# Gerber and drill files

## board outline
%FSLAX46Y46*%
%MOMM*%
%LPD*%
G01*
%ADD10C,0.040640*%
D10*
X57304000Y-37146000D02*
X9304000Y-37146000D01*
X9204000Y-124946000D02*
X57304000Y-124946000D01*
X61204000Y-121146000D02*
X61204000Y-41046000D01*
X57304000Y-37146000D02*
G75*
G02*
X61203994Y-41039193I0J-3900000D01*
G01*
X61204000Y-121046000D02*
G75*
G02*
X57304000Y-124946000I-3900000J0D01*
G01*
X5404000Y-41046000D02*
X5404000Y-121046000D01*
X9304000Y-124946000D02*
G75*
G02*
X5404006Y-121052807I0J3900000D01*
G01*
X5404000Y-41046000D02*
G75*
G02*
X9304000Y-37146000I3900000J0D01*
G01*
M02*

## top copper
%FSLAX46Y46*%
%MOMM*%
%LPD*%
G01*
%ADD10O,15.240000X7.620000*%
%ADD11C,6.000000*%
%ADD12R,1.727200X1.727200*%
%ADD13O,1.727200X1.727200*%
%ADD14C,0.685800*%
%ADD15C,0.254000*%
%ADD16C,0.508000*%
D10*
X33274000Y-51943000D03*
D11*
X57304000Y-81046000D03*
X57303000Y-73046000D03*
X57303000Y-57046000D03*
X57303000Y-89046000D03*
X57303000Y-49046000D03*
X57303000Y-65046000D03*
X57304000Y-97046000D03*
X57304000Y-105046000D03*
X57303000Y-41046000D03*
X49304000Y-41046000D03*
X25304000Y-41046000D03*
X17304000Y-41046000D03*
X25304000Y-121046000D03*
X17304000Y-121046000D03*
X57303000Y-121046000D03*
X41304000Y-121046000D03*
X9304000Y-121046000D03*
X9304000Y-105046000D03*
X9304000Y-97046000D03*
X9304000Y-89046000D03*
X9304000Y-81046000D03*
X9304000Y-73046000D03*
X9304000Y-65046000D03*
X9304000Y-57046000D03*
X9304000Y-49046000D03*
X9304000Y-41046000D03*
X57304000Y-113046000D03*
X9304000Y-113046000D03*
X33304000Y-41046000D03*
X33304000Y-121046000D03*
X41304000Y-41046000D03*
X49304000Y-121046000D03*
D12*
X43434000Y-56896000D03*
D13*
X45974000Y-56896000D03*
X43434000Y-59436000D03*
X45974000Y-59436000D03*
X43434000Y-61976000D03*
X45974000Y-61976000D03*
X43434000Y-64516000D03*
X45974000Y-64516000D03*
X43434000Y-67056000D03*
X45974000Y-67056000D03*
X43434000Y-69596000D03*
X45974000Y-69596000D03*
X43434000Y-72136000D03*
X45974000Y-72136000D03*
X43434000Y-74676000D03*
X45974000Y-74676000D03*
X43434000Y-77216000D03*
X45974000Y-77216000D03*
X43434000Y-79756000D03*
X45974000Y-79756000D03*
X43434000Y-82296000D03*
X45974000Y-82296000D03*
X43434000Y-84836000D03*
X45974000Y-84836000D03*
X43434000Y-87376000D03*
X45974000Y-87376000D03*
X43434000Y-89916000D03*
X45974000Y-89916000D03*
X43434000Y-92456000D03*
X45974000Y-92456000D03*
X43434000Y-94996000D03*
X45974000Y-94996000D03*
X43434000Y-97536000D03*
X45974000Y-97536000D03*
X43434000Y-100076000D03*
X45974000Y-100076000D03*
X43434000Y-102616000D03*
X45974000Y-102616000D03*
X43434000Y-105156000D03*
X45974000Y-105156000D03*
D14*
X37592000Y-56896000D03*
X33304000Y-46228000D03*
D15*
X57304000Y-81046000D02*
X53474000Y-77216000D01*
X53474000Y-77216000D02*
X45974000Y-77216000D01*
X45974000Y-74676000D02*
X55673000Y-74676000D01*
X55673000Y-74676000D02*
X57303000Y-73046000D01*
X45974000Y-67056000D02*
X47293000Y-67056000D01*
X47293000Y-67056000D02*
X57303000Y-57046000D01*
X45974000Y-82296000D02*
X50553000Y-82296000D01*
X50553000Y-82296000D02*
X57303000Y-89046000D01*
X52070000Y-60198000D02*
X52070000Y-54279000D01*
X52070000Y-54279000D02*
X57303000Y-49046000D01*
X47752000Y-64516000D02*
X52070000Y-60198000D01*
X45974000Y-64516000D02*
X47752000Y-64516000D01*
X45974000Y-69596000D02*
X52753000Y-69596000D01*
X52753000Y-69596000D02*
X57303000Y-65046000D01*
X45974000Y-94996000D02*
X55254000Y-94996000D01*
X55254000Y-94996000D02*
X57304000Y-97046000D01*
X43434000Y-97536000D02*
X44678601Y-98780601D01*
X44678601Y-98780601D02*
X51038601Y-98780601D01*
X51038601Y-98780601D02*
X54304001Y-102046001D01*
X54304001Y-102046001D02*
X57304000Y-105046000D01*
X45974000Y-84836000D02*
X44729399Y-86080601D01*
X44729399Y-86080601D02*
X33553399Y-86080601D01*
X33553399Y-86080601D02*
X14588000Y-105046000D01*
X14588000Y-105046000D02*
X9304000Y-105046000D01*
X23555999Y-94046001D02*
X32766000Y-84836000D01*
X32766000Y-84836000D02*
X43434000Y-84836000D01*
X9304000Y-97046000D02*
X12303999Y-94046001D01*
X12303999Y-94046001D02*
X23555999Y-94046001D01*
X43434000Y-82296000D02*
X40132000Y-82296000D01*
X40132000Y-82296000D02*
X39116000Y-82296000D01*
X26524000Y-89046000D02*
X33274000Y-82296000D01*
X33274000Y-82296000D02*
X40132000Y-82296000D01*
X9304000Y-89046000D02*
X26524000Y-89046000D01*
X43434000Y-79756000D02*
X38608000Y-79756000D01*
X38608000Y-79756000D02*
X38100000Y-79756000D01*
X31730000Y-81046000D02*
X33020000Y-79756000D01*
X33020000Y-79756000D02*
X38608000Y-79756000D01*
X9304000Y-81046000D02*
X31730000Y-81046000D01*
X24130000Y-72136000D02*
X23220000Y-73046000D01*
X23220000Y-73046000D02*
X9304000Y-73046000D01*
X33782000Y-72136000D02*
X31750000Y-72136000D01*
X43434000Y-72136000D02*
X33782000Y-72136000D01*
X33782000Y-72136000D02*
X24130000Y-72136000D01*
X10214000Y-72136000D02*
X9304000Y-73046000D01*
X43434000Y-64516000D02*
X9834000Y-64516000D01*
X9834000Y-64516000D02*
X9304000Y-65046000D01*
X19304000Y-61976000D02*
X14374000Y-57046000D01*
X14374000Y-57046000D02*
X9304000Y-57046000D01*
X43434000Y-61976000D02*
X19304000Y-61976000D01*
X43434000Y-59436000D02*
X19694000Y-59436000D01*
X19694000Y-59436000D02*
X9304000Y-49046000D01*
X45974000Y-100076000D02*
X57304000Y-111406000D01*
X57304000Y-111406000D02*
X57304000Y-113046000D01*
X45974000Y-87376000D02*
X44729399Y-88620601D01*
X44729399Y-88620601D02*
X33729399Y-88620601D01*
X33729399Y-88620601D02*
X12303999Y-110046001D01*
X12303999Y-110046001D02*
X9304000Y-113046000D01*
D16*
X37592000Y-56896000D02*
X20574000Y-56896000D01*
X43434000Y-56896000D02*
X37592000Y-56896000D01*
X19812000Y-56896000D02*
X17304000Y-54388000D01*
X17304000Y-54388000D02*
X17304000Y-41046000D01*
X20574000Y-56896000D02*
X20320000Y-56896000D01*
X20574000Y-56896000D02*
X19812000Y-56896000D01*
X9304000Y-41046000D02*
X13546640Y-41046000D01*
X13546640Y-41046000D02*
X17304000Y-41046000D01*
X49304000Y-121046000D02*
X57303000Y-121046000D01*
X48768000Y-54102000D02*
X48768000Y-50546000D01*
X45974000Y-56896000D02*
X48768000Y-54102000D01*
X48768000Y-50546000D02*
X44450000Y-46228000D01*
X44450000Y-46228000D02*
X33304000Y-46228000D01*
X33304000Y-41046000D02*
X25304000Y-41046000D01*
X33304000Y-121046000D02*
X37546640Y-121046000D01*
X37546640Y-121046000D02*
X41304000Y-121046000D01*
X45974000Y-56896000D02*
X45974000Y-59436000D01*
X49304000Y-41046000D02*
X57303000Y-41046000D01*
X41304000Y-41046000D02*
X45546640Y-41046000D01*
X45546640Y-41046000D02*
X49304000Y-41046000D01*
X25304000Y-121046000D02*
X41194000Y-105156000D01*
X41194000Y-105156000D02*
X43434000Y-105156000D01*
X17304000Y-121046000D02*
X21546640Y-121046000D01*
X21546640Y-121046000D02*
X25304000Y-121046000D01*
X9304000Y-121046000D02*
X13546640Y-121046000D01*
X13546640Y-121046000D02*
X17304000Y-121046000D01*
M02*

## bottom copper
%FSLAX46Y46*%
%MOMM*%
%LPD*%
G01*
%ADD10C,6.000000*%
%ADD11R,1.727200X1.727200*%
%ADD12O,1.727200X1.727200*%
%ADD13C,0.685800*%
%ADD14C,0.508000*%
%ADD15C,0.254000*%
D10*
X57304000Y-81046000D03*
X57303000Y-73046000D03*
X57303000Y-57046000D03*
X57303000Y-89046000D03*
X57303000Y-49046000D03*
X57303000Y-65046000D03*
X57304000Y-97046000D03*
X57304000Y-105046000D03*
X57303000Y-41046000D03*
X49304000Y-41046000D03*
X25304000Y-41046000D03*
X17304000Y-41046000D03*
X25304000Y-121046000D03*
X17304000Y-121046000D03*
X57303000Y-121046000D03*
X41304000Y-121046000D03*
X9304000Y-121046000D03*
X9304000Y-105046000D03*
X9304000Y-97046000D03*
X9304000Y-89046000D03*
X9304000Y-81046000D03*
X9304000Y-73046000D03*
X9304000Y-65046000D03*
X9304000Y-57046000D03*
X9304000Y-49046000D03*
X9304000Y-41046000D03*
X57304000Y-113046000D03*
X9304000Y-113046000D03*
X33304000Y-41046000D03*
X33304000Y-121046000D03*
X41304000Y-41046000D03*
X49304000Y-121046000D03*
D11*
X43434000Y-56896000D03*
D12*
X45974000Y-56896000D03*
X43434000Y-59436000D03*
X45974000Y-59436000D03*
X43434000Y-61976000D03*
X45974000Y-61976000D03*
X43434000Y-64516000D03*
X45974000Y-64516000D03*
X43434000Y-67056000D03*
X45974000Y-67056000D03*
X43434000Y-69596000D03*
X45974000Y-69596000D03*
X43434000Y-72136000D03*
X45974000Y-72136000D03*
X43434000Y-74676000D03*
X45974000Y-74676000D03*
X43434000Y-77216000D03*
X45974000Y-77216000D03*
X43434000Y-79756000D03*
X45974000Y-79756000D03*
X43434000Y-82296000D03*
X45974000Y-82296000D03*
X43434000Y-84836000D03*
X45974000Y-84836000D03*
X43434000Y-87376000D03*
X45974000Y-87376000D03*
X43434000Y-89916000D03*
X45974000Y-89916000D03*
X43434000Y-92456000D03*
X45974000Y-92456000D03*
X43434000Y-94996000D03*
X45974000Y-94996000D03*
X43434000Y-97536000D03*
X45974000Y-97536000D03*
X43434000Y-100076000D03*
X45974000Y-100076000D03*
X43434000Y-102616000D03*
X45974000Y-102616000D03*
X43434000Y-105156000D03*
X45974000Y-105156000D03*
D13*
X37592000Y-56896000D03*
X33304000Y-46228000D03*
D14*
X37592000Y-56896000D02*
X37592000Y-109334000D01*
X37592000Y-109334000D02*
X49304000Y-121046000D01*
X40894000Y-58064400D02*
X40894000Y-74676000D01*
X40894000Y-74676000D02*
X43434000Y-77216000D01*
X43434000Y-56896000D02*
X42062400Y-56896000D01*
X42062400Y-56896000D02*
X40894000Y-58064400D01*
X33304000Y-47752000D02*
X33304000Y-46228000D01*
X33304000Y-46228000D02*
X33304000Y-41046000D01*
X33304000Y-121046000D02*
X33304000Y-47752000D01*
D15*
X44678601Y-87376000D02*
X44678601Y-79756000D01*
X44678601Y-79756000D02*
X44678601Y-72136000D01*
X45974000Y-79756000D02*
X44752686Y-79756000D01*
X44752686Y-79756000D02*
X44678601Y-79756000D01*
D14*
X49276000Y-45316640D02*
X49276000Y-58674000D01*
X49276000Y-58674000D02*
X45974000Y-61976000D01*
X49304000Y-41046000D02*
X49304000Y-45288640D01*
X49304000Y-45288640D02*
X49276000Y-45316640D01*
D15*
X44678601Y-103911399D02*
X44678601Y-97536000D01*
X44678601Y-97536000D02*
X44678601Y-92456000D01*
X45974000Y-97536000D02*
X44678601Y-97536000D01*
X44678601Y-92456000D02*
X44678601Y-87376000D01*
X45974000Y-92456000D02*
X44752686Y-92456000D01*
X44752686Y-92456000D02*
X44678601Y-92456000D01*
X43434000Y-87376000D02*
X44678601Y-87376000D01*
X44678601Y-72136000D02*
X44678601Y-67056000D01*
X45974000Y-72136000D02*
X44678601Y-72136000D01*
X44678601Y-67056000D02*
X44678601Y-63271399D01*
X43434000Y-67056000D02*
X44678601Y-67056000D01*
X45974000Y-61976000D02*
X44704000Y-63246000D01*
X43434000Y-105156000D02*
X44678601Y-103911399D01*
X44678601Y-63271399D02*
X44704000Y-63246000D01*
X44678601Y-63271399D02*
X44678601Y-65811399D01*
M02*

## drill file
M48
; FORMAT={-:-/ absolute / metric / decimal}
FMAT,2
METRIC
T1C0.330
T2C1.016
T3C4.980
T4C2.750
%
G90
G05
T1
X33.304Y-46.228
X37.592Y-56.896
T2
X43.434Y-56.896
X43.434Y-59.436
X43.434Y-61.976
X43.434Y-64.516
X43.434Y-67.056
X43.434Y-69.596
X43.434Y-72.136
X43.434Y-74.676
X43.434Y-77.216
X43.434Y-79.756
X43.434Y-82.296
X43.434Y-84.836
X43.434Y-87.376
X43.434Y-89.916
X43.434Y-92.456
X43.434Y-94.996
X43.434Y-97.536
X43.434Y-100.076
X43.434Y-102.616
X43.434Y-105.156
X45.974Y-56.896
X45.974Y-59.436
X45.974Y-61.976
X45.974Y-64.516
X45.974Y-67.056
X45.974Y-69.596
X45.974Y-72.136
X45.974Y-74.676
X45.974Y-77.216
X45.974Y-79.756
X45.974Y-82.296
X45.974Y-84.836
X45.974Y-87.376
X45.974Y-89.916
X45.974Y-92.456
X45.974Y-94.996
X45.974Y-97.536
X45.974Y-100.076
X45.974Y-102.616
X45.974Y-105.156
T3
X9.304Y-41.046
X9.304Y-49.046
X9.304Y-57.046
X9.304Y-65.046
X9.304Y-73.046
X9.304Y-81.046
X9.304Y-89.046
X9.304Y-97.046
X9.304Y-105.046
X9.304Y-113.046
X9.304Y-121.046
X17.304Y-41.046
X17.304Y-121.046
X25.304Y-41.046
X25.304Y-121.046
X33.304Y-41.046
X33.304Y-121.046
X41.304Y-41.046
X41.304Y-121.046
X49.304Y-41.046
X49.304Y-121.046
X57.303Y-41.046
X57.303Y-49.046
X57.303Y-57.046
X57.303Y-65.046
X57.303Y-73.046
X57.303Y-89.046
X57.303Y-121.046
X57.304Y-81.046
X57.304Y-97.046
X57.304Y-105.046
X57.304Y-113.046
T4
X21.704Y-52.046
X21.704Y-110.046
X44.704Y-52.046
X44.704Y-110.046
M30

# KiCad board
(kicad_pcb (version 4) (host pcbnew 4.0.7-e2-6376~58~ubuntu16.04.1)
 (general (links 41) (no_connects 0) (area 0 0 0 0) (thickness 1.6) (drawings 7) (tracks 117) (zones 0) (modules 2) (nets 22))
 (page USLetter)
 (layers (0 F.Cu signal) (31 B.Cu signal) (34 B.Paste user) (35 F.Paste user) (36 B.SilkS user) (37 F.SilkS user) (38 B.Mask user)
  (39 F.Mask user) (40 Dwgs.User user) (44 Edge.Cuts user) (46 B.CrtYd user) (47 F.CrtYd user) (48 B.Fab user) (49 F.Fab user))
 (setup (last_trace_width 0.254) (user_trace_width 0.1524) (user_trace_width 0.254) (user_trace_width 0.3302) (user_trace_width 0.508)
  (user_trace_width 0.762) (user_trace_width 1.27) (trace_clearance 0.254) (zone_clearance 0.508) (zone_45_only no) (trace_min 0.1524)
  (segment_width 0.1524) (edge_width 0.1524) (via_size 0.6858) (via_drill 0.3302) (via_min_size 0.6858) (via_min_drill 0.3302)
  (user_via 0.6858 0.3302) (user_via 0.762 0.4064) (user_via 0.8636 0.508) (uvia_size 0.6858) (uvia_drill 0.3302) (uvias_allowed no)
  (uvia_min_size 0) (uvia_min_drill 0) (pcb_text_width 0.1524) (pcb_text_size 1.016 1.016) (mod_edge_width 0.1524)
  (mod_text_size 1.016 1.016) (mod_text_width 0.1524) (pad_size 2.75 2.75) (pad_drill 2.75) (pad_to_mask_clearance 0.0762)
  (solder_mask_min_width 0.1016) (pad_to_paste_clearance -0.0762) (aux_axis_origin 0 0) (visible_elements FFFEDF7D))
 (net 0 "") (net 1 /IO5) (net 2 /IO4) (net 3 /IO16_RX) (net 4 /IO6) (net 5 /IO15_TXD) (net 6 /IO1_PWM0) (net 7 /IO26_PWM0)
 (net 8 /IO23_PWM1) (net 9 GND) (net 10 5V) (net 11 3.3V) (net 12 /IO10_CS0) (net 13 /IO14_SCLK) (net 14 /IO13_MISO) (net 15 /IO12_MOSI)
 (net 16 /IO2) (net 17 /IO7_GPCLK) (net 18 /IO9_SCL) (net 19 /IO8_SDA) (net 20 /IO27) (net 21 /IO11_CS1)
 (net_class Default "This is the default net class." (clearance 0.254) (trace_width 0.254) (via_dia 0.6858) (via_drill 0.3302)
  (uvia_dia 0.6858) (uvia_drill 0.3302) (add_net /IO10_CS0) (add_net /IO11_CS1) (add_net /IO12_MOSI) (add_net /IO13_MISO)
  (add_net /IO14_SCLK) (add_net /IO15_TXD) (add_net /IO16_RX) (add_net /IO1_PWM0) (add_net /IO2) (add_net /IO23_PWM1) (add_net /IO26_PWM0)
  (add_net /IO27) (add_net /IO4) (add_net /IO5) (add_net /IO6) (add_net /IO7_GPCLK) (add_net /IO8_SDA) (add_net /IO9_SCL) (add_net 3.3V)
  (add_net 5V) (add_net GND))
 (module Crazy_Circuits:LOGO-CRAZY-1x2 (layer F.Cu) (at 33.274 55.88)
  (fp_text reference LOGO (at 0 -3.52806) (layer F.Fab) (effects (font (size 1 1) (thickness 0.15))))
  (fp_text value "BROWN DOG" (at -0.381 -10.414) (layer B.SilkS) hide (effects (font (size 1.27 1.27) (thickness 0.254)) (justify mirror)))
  (pad BG smd oval (at 0 -3.937) (size 15.24 7.62) (layers F.Cu)))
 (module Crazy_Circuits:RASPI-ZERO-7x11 (layer F.Cu) (at 9.204 41.546)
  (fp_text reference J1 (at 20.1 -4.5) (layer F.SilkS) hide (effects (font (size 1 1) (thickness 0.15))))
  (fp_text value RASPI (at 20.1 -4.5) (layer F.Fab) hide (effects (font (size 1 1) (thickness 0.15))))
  (fp_line (start 48.1 -4.4) (end 0.1 -4.4) (layer Edge.Cuts) (width 0.04064))
  (fp_line (start 0 83.4) (end 48.1 83.4) (layer Edge.Cuts) (width 0.04064))
  (fp_line (start 52 79.6) (end 52 -0.5) (layer Edge.Cuts) (width 0.04064))
  (fp_arc (start 48.1 -0.5) (end 48.1 -4.4) (angle 89.9) (layer Edge.Cuts) (width 0.04064))
  (fp_arc (start 48.1 79.5) (end 52 79.5) (angle 90) (layer Edge.Cuts) (width 0.04064))
  (fp_line (start -3.8 -0.5) (end -3.8 79.5) (layer Edge.Cuts) (width 0.04064))
  (fp_arc (start 0.1 79.5) (end 0.1 83.4) (angle 89.9) (layer Edge.Cuts) (width 0.04064))
  (fp_arc (start 0.1 -0.5) (end -3.8 -0.5) (angle 90) (layer Edge.Cuts) (width 0.04064))
  (pad 18 thru_hole circle (at 48.1 39.5 270) (size 6 6) (drill 4.98) (layers *.Cu *.Mask) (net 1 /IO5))
  (pad 16 thru_hole circle (at 48.099 31.5 270) (size 6 6) (drill 4.98) (layers *.Cu *.Mask) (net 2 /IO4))
  (pad 10 thru_hole circle (at 48.099 15.5 270) (size 6 6) (drill 4.98) (layers *.Cu *.Mask) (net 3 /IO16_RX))
  (pad 22 thru_hole circle (at 48.099 47.5 270) (size 6 6) (drill 4.98) (layers *.Cu *.Mask) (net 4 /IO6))
  (pad 8 thru_hole circle (at 48.099 7.5 270) (size 6 6) (drill 4.98) (layers *.Cu *.Mask) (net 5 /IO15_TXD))
  (pad 12 thru_hole circle (at 48.099 23.5 270) (size 6 6) (drill 4.98) (layers *.Cu *.Mask) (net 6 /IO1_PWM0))
  (pad 32 thru_hole circle (at 48.1 55.5 270) (size 6 6) (drill 4.98) (layers *.Cu *.Mask) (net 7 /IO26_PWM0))
  (pad 33 thru_hole circle (at 48.1 63.5 270) (size 6 6) (drill 4.98) (layers *.Cu *.Mask) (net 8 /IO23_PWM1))
  (pad 6 thru_hole circle (at 48.099 -0.5 270) (size 6 6) (drill 4.98) (layers *.Cu *.Mask) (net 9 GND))
  (pad 6 thru_hole circle (at 40.1 -0.5 270) (size 6 6) (drill 4.98) (layers *.Cu *.Mask) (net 9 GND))
  (pad 2 thru_hole circle (at 16.1 -0.5 270) (size 6 6) (drill 4.98) (layers *.Cu *.Mask) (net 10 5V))
  (pad 1 thru_hole circle (at 8.1 -0.5 270) (size 6 6) (drill 4.98) (layers *.Cu *.Mask) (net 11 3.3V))
  (pad 6 thru_hole circle (at 16.1 79.5 270) (size 6 6) (drill 4.98) (layers *.Cu *.Mask) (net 9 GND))
  (pad 6 thru_hole circle (at 8.1 79.5 270) (size 6 6) (drill 4.98) (layers *.Cu *.Mask) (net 9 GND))
  (pad 1 thru_hole circle (at 48.099 79.5 270) (size 6 6) (drill 4.98) (layers *.Cu *.Mask) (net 11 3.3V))
  (pad 2 thru_hole circle (at 32.1 79.5 270) (size 6 6) (drill 4.98) (layers *.Cu *.Mask) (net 10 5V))
  (pad 6 thru_hole circle (at 0.1 79.5 270) (size 6 6) (drill 4.98) (layers *.Cu *.Mask) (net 9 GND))
  (pad 24 thru_hole circle (at 0.1 63.5 270) (size 6 6) (drill 4.98) (layers *.Cu *.Mask) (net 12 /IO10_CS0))
  (pad 23 thru_hole circle (at 0.1 55.5 270) (size 6 6) (drill 4.98) (layers *.Cu *.Mask) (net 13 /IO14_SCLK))
  (pad 21 thru_hole circle (at 0.1 47.5 270) (size 6 6) (drill 4.98) (layers *.Cu *.Mask) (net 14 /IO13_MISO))
  (pad 19 thru_hole circle (at 0.1 39.5 270) (size 6 6) (drill 4.98) (layers *.Cu *.Mask) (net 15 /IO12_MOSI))
  (pad 13 thru_hole circle (at 0.1 31.5 270) (size 6 6) (drill 4.98) (layers *.Cu *.Mask) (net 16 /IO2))
  (pad 7 thru_hole circle (at 0.1 23.5 270) (size 6 6) (drill 4.98) (layers *.Cu *.Mask) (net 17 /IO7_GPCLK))
  (pad 5 thru_hole circle (at 0.1 15.5 270) (size 6 6) (drill 4.98) (layers *.Cu *.Mask) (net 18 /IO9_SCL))
  (pad 3 thru_hole circle (at 0.1 7.5 270) (size 6 6) (drill 4.98) (layers *.Cu *.Mask) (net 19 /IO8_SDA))
  (pad 1 thru_hole circle (at 0.1 -0.5 270) (size 6 6) (drill 4.98) (layers *.Cu *.Mask) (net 11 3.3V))
  (pad 36 thru_hole circle (at 48.1 71.5 270) (size 6 6) (drill 4.98) (layers *.Cu *.Mask) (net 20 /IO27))
  (pad 26 thru_hole circle (at 0.1 71.5 270) (size 6 6) (drill 4.98) (layers *.Cu *.Mask) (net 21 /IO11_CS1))
  (pad 2 thru_hole circle (at 24.1 -0.5 270) (size 6 6) (drill 4.98) (layers *.Cu *.Mask) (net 10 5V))
  (pad 2 thru_hole circle (at 24.1 79.5 270) (size 6 6) (drill 4.98) (layers *.Cu *.Mask) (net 10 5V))
  (pad 6 thru_hole circle (at 32.1 -0.5 270) (size 6 6) (drill 4.98) (layers *.Cu *.Mask) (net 9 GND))
  (pad 1 thru_hole circle (at 40.1 79.5 270) (size 6 6) (drill 4.98) (layers *.Cu *.Mask) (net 11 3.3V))
  (pad "" np_thru_hole circle (at 12.5 10.5 270) (size 2.75 2.75) (drill 2.75) (layers *.Cu) (solder_mask_margin 1.75) (clearance 1.75))
  (pad "" np_thru_hole circle (at 35.5 10.5 270) (size 2.75 2.75) (drill 2.75) (layers *.Cu) (solder_mask_margin 1.75) (clearance 1.75))
  (pad "" np_thru_hole circle (at 35.5 68.5 90) (size 2.75 2.75) (drill 2.75) (layers *.Cu) (solder_mask_margin 1.75) (clearance 1.75))
  (pad "" np_thru_hole circle (at 12.5 68.5 90) (size 2.75 2.75) (drill 2.75) (layers *.Cu) (solder_mask_margin 1.75) (clearance 1.75))
  (pad 1 thru_hole rect (at 34.23 15.35) (size 1.7272 1.7272) (drill 1.016) (layers *.Cu *.Mask F.SilkS) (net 11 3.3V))
  (pad 2 thru_hole oval (at 36.77 15.35) (size 1.7272 1.7272) (drill 1.016) (layers *.Cu *.Mask F.SilkS) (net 10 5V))
  (pad 3 thru_hole oval (at 34.23 17.89) (size 1.7272 1.7272) (drill 1.016) (layers *.Cu *.Mask F.SilkS) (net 19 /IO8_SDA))
  (pad 4 thru_hole oval (at 36.77 17.89) (size 1.7272 1.7272) (drill 1.016) (layers *.Cu *.Mask F.SilkS) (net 10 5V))
  (pad 5 thru_hole oval (at 34.23 20.43) (size 1.7272 1.7272) (drill 1.016) (layers *.Cu *.Mask F.SilkS) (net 18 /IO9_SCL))
  (pad 6 thru_hole oval (at 36.77 20.43) (size 1.7272 1.7272) (drill 1.016) (layers *.Cu *.Mask F.SilkS) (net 9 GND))
  (pad 7 thru_hole oval (at 34.23 22.97) (size 1.7272 1.7272) (drill 1.016) (layers *.Cu *.Mask F.SilkS) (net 17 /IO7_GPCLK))
  (pad 8 thru_hole oval (at 36.77 22.97) (size 1.7272 1.7272) (drill 1.016) (layers *.Cu *.Mask F.SilkS) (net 5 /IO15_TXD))
  (pad 9 thru_hole oval (at 34.23 25.51) (size 1.7272 1.7272) (drill 1.016) (layers *.Cu *.Mask F.SilkS) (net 9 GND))
  (pad 10 thru_hole oval (at 36.77 25.51) (size 1.7272 1.7272) (drill 1.016) (layers *.Cu *.Mask F.SilkS) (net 3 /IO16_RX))
  (pad 11 thru_hole oval (at 34.23 28.05) (size 1.7272 1.7272) (drill 1.016) (layers *.Cu *.Mask F.SilkS))
  (pad 12 thru_hole oval (at 36.77 28.05) (size 1.7272 1.7272) (drill 1.016) (layers *.Cu *.Mask F.SilkS) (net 6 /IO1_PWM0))
  (pad 13 thru_hole oval (at 34.23 30.59) (size 1.7272 1.7272) (drill 1.016) (layers *.Cu *.Mask F.SilkS) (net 16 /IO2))
  (pad 14 thru_hole oval (at 36.77 30.59) (size 1.7272 1.7272) (drill 1.016) (layers *.Cu *.Mask F.SilkS) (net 9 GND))
  (pad 15 thru_hole oval (at 34.23 33.13) (size 1.7272 1.7272) (drill 1.016) (layers *.Cu *.Mask F.SilkS))
  (pad 16 thru_hole oval (at 36.77 33.13) (size 1.7272 1.7272) (drill 1.016) (layers *.Cu *.Mask F.SilkS) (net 2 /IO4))
  (pad 17 thru_hole oval (at 34.23 35.67) (size 1.7272 1.7272) (drill 1.016) (layers *.Cu *.Mask F.SilkS) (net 11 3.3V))
  (pad 18 thru_hole oval (at 36.77 35.67) (size 1.7272 1.7272) (drill 1.016) (layers *.Cu *.Mask F.SilkS) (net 1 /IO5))
  (pad 19 thru_hole oval (at 34.23 38.21) (size 1.7272 1.7272) (drill 1.016) (layers *.Cu *.Mask F.SilkS) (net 15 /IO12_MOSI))
  (pad 20 thru_hole oval (at 36.77 38.21) (size 1.7272 1.7272) (drill 1.016) (layers *.Cu *.Mask F.SilkS) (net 9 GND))
  (pad 21 thru_hole oval (at 34.23 40.75) (size 1.7272 1.7272) (drill 1.016) (layers *.Cu *.Mask F.SilkS) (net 14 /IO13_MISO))
  (pad 22 thru_hole oval (at 36.77 40.75) (size 1.7272 1.7272) (drill 1.016) (layers *.Cu *.Mask F.SilkS) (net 4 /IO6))
  (pad 23 thru_hole oval (at 34.23 43.29) (size 1.7272 1.7272) (drill 1.016) (layers *.Cu *.Mask F.SilkS) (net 13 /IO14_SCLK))
  (pad 24 thru_hole oval (at 36.77 43.29) (size 1.7272 1.7272) (drill 1.016) (layers *.Cu *.Mask F.SilkS) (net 12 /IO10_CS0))
  (pad 25 thru_hole oval (at 34.23 45.83) (size 1.7272 1.7272) (drill 1.016) (layers *.Cu *.Mask F.SilkS) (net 9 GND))
  (pad 26 thru_hole oval (at 36.77 45.83) (size 1.7272 1.7272) (drill 1.016) (layers *.Cu *.Mask F.SilkS) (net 21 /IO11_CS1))
  (pad 27 thru_hole oval (at 34.23 48.37) (size 1.7272 1.7272) (drill 1.016) (layers *.Cu *.Mask F.SilkS))
  (pad 28 thru_hole oval (at 36.77 48.37) (size 1.7272 1.7272) (drill 1.016) (layers *.Cu *.Mask F.SilkS))
  (pad 29 thru_hole oval (at 34.23 50.91) (size 1.7272 1.7272) (drill 1.016) (layers *.Cu *.Mask F.SilkS))
  (pad 30 thru_hole oval (at 36.77 50.91) (size 1.7272 1.7272) (drill 1.016) (layers *.Cu *.Mask F.SilkS) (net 9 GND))
  (pad 31 thru_hole oval (at 34.23 53.45) (size 1.7272 1.7272) (drill 1.016) (layers *.Cu *.Mask F.SilkS))
  (pad 32 thru_hole oval (at 36.77 53.45) (size 1.7272 1.7272) (drill 1.016) (layers *.Cu *.Mask F.SilkS) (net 7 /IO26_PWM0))
  (pad 33 thru_hole oval (at 34.23 55.99) (size 1.7272 1.7272) (drill 1.016) (layers *.Cu *.Mask F.SilkS) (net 8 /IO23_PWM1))
  (pad 34 thru_hole oval (at 36.77 55.99) (size 1.7272 1.7272) (drill 1.016) (layers *.Cu *.Mask F.SilkS) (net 9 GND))
  (pad 35 thru_hole oval (at 34.23 58.53) (size 1.7272 1.7272) (drill 1.016) (layers *.Cu *.Mask F.SilkS))
  (pad 36 thru_hole oval (at 36.77 58.53) (size 1.7272 1.7272) (drill 1.016) (layers *.Cu *.Mask F.SilkS) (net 20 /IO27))
  (pad 37 thru_hole oval (at 34.23 61.07) (size 1.7272 1.7272) (drill 1.016) (layers *.Cu *.Mask F.SilkS))
  (pad 38 thru_hole oval (at 36.77 61.07) (size 1.7272 1.7272) (drill 1.016) (layers *.Cu *.Mask F.SilkS))
  (pad 39 thru_hole oval (at 34.23 63.61) (size 1.7272 1.7272) (drill 1.016) (layers *.Cu *.Mask F.SilkS) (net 9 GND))
  (pad 40 thru_hole oval (at 36.77 63.61) (size 1.7272 1.7272) (drill 1.016) (layers *.Cu *.Mask F.SilkS)))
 (segment (start 57.304 81.046) (end 53.474 77.216) (width 0.254) (layer F.Cu) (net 1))
 (segment (start 53.474 77.216) (end 45.974 77.216) (width 0.254) (layer F.Cu) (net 1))
 (segment (start 45.974 74.676) (end 55.673 74.676) (width 0.254) (layer F.Cu) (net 2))
 (segment (start 55.673 74.676) (end 57.303 73.046) (width 0.254) (layer F.Cu) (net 2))
 (segment (start 45.974 67.056) (end 47.293 67.056) (width 0.254) (layer F.Cu) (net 3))
 (segment (start 47.293 67.056) (end 57.303 57.046) (width 0.254) (layer F.Cu) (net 3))
 (segment (start 45.974 82.296) (end 50.553 82.296) (width 0.254) (layer F.Cu) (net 4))
 (segment (start 50.553 82.296) (end 57.303 89.046) (width 0.254) (layer F.Cu) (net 4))
 (segment (start 52.07 60.198) (end 52.07 54.279) (width 0.254) (layer F.Cu) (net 5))
 (segment (start 52.07 54.279) (end 57.303 49.046) (width 0.254) (layer F.Cu) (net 5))
 (segment (start 47.752 64.516) (end 52.07 60.198) (width 0.254) (layer F.Cu) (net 5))
 (segment (start 45.974 64.516) (end 47.752 64.516) (width 0.254) (layer F.Cu) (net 5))
 (segment (start 45.974 69.596) (end 52.753 69.596) (width 0.254) (layer F.Cu) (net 6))
 (segment (start 52.753 69.596) (end 57.303 65.046) (width 0.254) (layer F.Cu) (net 6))
 (segment (start 45.974 94.996) (end 55.254 94.996) (width 0.254) (layer F.Cu) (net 7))
 (segment (start 55.254 94.996) (end 57.304 97.046) (width 0.254) (layer F.Cu) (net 7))
 (segment (start 43.434 97.536) (end 44.678601 98.780601) (width 0.254) (layer F.Cu) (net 8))
 (segment (start 44.678601 98.780601) (end 51.038601 98.780601) (width 0.254) (layer F.Cu) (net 8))
 (segment (start 51.038601 98.780601) (end 54.304001 102.046001) (width 0.254) (layer F.Cu) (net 8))
 (segment (start 54.304001 102.046001) (end 57.304 105.046) (width 0.254) (layer F.Cu) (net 8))
 (segment (start 45.974 84.836) (end 44.729399 86.080601) (width 0.254) (layer F.Cu) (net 12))
 (segment (start 44.729399 86.080601) (end 33.553399 86.080601) (width 0.254) (layer F.Cu) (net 12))
 (segment (start 33.553399 86.080601) (end 14.588 105.046) (width 0.254) (layer F.Cu) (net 12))
 (segment (start 14.588 105.046) (end 9.304 105.046) (width 0.254) (layer F.Cu) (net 12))
 (segment (start 23.555999 94.046001) (end 32.766 84.836) (width 0.254) (layer F.Cu) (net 13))
 (segment (start 32.766 84.836) (end 43.434 84.836) (width 0.254) (layer F.Cu) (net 13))
 (segment (start 9.304 97.046) (end 12.303999 94.046001) (width 0.254) (layer F.Cu) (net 13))
 (segment (start 12.303999 94.046001) (end 23.555999 94.046001) (width 0.254) (layer F.Cu) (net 13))
 (segment (start 43.434 82.296) (end 40.132 82.296) (width 0.254) (layer F.Cu) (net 14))
 (segment (start 40.132 82.296) (end 39.116 82.296) (width 0.254) (layer F.Cu) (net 14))
 (segment (start 26.524 89.046) (end 33.274 82.296) (width 0.254) (layer F.Cu) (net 14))
 (segment (start 33.274 82.296) (end 40.132 82.296) (width 0.254) (layer F.Cu) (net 14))
 (segment (start 9.304 89.046) (end 26.524 89.046) (width 0.254) (layer F.Cu) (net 14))
 (segment (start 43.434 79.756) (end 38.608 79.756) (width 0.254) (layer F.Cu) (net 15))
 (segment (start 38.608 79.756) (end 38.1 79.756) (width 0.254) (layer F.Cu) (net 15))
 (segment (start 31.73 81.046) (end 33.02 79.756) (width 0.254) (layer F.Cu) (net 15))
 (segment (start 33.02 79.756) (end 38.608 79.756) (width 0.254) (layer F.Cu) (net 15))
 (segment (start 9.304 81.046) (end 31.73 81.046) (width 0.254) (layer F.Cu) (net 15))
 (segment (start 24.13 72.136) (end 23.22 73.046) (width 0.254) (layer F.Cu) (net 16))
 (segment (start 23.22 73.046) (end 9.304 73.046) (width 0.254) (layer F.Cu) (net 16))
 (segment (start 33.782 72.136) (end 31.75 72.136) (width 0.254) (layer F.Cu) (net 16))
 (segment (start 43.434 72.136) (end 33.782 72.136) (width 0.254) (layer F.Cu) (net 16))
 (segment (start 33.782 72.136) (end 24.13 72.136) (width 0.254) (layer F.Cu) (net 16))
 (segment (start 10.214 72.136) (end 9.304 73.046) (width 0.254) (layer F.Cu) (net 16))
 (segment (start 43.434 64.516) (end 9.834 64.516) (width 0.254) (layer F.Cu) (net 17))
 (segment (start 9.834 64.516) (end 9.304 65.046) (width 0.254) (layer F.Cu) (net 17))
 (segment (start 19.304 61.976) (end 14.374 57.046) (width 0.254) (layer F.Cu) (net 18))
 (segment (start 14.374 57.046) (end 9.304 57.046) (width 0.254) (layer F.Cu) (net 18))
 (segment (start 43.434 61.976) (end 19.304 61.976) (width 0.254) (layer F.Cu) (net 18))
 (segment (start 43.434 59.436) (end 19.694 59.436) (width 0.254) (layer F.Cu) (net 19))
 (segment (start 19.694 59.436) (end 9.304 49.046) (width 0.254) (layer F.Cu) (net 19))
 (segment (start 45.974 100.076) (end 57.304 111.406) (width 0.254) (layer F.Cu) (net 20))
 (segment (start 57.304 111.406) (end 57.304 113.046) (width 0.254) (layer F.Cu) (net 20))
 (segment (start 45.974 87.376) (end 44.729399 88.620601) (width 0.254) (layer F.Cu) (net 21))
 (segment (start 44.729399 88.620601) (end 33.729399 88.620601) (width 0.254) (layer F.Cu) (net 21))
 (segment (start 33.729399 88.620601) (end 12.303999 110.046001) (width 0.254) (layer F.Cu) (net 21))
 (segment (start 12.303999 110.046001) (end 9.304 113.046) (width 0.254) (layer F.Cu) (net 21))
 (segment (start 37.592 56.896) (end 37.592 109.334) (width 0.508) (layer B.Cu) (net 11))
 (segment (start 37.592 109.334) (end 49.304 121.046) (width 0.508) (layer B.Cu) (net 11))
 (segment (start 37.592 56.896) (end 20.574 56.896) (width 0.508) (layer F.Cu) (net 11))
 (segment (start 43.434 56.896) (end 37.592 56.896) (width 0.508) (layer F.Cu) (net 11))
 (via (at 37.592 56.896) (size 0.6858) (drill 0.3302) (layers F.Cu B.Cu) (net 11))
 (segment (start 19.812 56.896) (end 17.304 54.388) (width 0.508) (layer F.Cu) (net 11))
 (segment (start 17.304 54.388) (end 17.304 41.046) (width 0.508) (layer F.Cu) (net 11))
 (segment (start 20.574 56.896) (end 20.32 56.896) (width 0.508) (layer F.Cu) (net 11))
 (segment (start 20.574 56.896) (end 19.812 56.896) (width 0.508) (layer F.Cu) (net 11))
 (segment (start 9.304 41.046) (end 13.54664 41.046) (width 0.508) (layer F.Cu) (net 11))
 (segment (start 13.54664 41.046) (end 17.304 41.046) (width 0.508) (layer F.Cu) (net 11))
 (segment (start 49.304 121.046) (end 57.303 121.046) (width 0.508) (layer F.Cu) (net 11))
 (segment (start 40.894 58.0644) (end 40.894 74.676) (width 0.508) (layer B.Cu) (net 11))
 (segment (start 40.894 74.676) (end 43.434 77.216) (width 0.508) (layer B.Cu) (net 11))
 (segment (start 43.434 56.896) (end 42.0624 56.896) (width 0.508) (layer B.Cu) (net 11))
 (segment (start 42.0624 56.896) (end 40.894 58.0644) (width 0.508) (layer B.Cu) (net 11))
 (segment (start 33.304 47.752) (end 33.304 46.228) (width 0.508) (layer B.Cu) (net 10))
 (segment (start 33.304 46.228) (end 33.304 41.046) (width 0.508) (layer B.Cu) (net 10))
 (segment (start 48.768 54.102) (end 48.768 50.546) (width 0.508) (layer F.Cu) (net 10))
 (via (at 33.304 46.228) (size 0.6858) (drill 0.3302) (layers F.Cu B.Cu) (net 10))
 (segment (start 45.974 56.896) (end 48.768 54.102) (width 0.508) (layer F.Cu) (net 10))
 (segment (start 48.768 50.546) (end 44.45 46.228) (width 0.508) (layer F.Cu) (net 10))
 (segment (start 44.45 46.228) (end 33.304 46.228) (width 0.508) (layer F.Cu) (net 10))
 (segment (start 33.304 121.046) (end 33.304 47.752) (width 0.508) (layer B.Cu) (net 10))
 (segment (start 33.304 41.046) (end 25.304 41.046) (width 0.508) (layer F.Cu) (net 10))
 (segment (start 33.304 121.046) (end 37.54664 121.046) (width 0.508) (layer F.Cu) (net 10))
 (segment (start 37.54664 121.046) (end 41.304 121.046) (width 0.508) (layer F.Cu) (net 10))
 (segment (start 45.974 56.896) (end 45.974 59.436) (width 0.508) (layer F.Cu) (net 10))
 (segment (start 44.678601 87.376) (end 44.678601 79.756) (width 0.254) (layer B.Cu) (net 9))
 (segment (start 44.678601 79.756) (end 44.678601 72.136) (width 0.254) (layer B.Cu) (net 9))
 (segment (start 45.974 79.756) (end 44.752686 79.756) (width 0.254) (layer B.Cu) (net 9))
 (segment (start 44.752686 79.756) (end 44.678601 79.756) (width 0.254) (layer B.Cu) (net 9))
 (segment (start 49.276 45.31664) (end 49.276 58.674) (width 0.508) (layer B.Cu) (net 9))
 (segment (start 49.276 58.674) (end 45.974 61.976) (width 0.508) (layer B.Cu) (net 9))
 (segment (start 49.304 41.046) (end 49.304 45.28864) (width 0.508) (layer B.Cu) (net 9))
 (segment (start 49.304 45.28864) (end 49.276 45.31664) (width 0.508) (layer B.Cu) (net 9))
 (segment (start 49.304 41.046) (end 57.303 41.046) (width 0.508) (layer F.Cu) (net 9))
 (segment (start 41.304 41.046) (end 45.54664 41.046) (width 0.508) (layer F.Cu) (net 9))
 (segment (start 45.54664 41.046) (end 49.304 41.046) (width 0.508) (layer F.Cu) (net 9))
 (segment (start 25.304 121.046) (end 41.194 105.156) (width 0.508) (layer F.Cu) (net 9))
 (segment (start 41.194 105.156) (end 43.434 105.156) (width 0.508) (layer F.Cu) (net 9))
 (segment (start 17.304 121.046) (end 21.54664 121.046) (width 0.508) (layer F.Cu) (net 9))
 (segment (start 21.54664 121.046) (end 25.304 121.046) (width 0.508) (layer F.Cu) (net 9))
 (segment (start 9.304 121.046) (end 13.54664 121.046) (width 0.508) (layer F.Cu) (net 9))
 (segment (start 13.54664 121.046) (end 17.304 121.046) (width 0.508) (layer F.Cu) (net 9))
 (segment (start 44.678601 103.911399) (end 44.678601 97.536) (width 0.254) (layer B.Cu) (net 9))
 (segment (start 44.678601 97.536) (end 44.678601 92.456) (width 0.254) (layer B.Cu) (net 9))
 (segment (start 45.974 97.536) (end 44.678601 97.536) (width 0.254) (layer B.Cu) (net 9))
 (segment (start 44.678601 92.456) (end 44.678601 87.376) (width 0.254) (layer B.Cu) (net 9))
 (segment (start 45.974 92.456) (end 44.752686 92.456) (width 0.254) (layer B.Cu) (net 9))
 (segment (start 44.752686 92.456) (end 44.678601 92.456) (width 0.254) (layer B.Cu) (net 9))
 (segment (start 43.434 87.376) (end 44.678601 87.376) (width 0.254) (layer B.Cu) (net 9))
 (segment (start 44.678601 72.136) (end 44.678601 67.056) (width 0.254) (layer B.Cu) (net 9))
 (segment (start 45.974 72.136) (end 44.678601 72.136) (width 0.254) (layer B.Cu) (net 9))
 (segment (start 44.678601 67.056) (end 44.678601 63.271399) (width 0.254) (layer B.Cu) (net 9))
 (segment (start 43.434 67.056) (end 44.678601 67.056) (width 0.254) (layer B.Cu) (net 9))
 (segment (start 45.974 61.976) (end 44.704 63.246) (width 0.254) (layer B.Cu) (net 9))
 (segment (start 43.434 105.156) (end 44.678601 103.911399) (width 0.254) (layer B.Cu) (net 9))
 (segment (start 44.678601 63.271399) (end 44.704 63.246) (width 0.254) (layer B.Cu) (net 9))
 (segment (start 44.678601 63.271399) (end 44.678601 65.811399) (width 0.254) (layer B.Cu) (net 9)))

